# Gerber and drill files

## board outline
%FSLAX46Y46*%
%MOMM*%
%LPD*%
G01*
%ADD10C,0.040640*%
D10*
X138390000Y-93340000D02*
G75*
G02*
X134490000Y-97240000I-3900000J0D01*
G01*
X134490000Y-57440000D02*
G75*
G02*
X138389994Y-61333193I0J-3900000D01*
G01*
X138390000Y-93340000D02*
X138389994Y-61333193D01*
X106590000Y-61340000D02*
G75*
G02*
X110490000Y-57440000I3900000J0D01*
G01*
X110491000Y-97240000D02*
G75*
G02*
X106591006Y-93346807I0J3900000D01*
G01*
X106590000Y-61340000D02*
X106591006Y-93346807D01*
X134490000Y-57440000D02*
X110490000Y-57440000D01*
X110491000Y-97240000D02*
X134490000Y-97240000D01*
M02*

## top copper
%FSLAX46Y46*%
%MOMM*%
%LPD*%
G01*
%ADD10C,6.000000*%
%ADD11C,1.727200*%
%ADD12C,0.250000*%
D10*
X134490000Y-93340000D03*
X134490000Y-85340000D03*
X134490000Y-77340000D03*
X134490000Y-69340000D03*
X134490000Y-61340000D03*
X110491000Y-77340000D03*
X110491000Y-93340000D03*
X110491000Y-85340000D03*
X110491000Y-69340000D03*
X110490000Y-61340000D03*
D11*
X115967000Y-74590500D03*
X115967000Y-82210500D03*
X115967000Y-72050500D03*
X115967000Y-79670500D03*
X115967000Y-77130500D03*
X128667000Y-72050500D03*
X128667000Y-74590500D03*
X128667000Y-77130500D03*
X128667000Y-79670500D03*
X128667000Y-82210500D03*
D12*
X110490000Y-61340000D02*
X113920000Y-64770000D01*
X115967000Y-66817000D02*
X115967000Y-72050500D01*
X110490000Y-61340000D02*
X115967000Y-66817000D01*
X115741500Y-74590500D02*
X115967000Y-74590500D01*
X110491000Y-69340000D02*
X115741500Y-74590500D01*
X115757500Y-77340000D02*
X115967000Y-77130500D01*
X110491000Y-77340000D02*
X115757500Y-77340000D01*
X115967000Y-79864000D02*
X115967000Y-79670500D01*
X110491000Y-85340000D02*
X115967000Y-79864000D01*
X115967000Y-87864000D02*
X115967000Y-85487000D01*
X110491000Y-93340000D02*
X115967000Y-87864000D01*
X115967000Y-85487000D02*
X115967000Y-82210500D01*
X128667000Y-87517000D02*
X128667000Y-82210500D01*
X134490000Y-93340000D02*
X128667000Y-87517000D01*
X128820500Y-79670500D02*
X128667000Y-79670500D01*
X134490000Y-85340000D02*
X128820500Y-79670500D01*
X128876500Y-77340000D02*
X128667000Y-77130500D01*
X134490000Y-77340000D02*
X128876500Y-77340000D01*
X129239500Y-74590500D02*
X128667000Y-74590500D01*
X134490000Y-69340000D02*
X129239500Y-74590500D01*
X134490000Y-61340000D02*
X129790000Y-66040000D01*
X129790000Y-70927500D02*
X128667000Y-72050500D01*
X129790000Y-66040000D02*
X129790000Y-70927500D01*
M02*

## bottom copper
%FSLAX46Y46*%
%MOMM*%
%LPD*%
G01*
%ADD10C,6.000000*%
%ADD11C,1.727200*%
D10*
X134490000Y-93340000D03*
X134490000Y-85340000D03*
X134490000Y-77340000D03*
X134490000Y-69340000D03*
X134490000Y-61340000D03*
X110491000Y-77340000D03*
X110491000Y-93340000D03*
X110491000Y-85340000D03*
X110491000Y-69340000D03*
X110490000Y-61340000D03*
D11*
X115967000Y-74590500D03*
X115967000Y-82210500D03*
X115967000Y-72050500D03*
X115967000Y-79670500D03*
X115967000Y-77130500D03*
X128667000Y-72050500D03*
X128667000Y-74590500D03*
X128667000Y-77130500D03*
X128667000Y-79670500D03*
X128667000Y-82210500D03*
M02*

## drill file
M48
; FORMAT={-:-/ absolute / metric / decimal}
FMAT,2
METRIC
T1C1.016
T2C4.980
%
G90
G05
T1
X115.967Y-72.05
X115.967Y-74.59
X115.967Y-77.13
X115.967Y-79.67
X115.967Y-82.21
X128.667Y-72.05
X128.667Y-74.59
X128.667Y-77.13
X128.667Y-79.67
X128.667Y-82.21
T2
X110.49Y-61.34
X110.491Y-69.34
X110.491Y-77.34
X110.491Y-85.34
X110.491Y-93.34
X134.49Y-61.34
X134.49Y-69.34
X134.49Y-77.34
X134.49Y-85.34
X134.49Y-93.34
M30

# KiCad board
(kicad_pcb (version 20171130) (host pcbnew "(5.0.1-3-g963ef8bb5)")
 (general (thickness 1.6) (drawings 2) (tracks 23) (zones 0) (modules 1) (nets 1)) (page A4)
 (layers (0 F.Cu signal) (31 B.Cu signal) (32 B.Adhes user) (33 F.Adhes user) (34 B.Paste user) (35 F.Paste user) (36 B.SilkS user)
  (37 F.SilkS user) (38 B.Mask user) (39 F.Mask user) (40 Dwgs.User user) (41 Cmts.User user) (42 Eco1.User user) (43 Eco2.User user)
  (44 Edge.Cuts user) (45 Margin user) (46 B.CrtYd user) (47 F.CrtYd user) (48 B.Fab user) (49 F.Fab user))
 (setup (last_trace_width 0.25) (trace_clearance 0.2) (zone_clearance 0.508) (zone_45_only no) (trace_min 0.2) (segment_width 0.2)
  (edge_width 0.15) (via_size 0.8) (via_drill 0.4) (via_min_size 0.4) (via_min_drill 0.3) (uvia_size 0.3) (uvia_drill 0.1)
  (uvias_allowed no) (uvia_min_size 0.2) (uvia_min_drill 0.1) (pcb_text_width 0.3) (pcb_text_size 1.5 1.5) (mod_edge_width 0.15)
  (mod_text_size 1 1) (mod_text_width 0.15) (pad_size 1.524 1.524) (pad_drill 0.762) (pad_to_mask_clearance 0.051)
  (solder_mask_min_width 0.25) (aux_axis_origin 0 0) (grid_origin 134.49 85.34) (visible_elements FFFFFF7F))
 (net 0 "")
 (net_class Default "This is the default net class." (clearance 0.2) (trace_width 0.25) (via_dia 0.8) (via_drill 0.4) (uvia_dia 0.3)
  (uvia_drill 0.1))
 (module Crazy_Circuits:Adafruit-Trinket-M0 (layer F.Cu) (at 110.49 53.34)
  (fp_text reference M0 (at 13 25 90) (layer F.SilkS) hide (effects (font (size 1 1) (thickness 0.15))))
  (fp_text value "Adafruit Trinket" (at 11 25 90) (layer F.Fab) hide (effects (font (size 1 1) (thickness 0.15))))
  (fp_arc (start 24 40) (end 27.9 40) (angle 90) (layer Edge.Cuts) (width 0.04064))
  (fp_arc (start 24 8) (end 24 4.1) (angle 89.89999678) (layer Edge.Cuts) (width 0.04064))
  (fp_line (start 27.9 40) (end 27.899994 7.993193) (layer Edge.Cuts) (width 0.04064))
  (fp_arc (start 0 8) (end -3.9 8) (angle 90) (layer Edge.Cuts) (width 0.04064))
  (fp_arc (start 0.001 40) (end 0.001 43.9) (angle 89.89999678) (layer Edge.Cuts) (width 0.04064))
  (fp_line (start -3.9 8) (end -3.898994 40.006807) (layer Edge.Cuts) (width 0.04064))
  (fp_line (start 24 4.1) (end 0 4.1) (layer Edge.Cuts) (width 0.04064))
  (fp_line (start 0.001 43.9) (end 24 43.9) (layer Edge.Cuts) (width 0.04064))
  (pad Bat thru_hole circle (at 24 40 90) (size 6 6) (drill 4.98) (layers *.Cu *.Mask))
  (pad Gnd thru_hole circle (at 24 32 90) (size 6 6) (drill 4.98) (layers *.Cu *.Mask))
  (pad 4 thru_hole circle (at 24 24 90) (size 6 6) (drill 4.98) (layers *.Cu *.Mask))
  (pad 3 thru_hole circle (at 24 16 90) (size 6 6) (drill 4.98) (layers *.Cu *.Mask))
  (pad Rst thru_hole circle (at 24 8 90) (size 6 6) (drill 4.98) (layers *.Cu *.Mask))
  (pad 1 thru_hole circle (at 0.001 24 90) (size 6 6) (drill 4.98) (layers *.Cu *.Mask))
  (pad USB thru_hole circle (at 0.001 40 90) (size 6 6) (drill 4.98) (layers *.Cu *.Mask))
  (pad 0 thru_hole circle (at 0.001 32 90) (size 6 6) (drill 4.98) (layers *.Cu *.Mask))
  (pad 2 thru_hole circle (at 0.001 16 90) (size 6 6) (drill 4.98) (layers *.Cu *.Mask))
  (pad 3V thru_hole circle (at 0 8 90) (size 6 6) (drill 4.98) (layers *.Cu *.Mask))
  (pad 2 thru_hole circle (at 5.477 21.2505 180) (size 1.7272 1.7272) (drill 1.016) (layers *.Cu *.Mask F.SilkS))
  (pad USB thru_hole circle (at 5.477 28.8705 180) (size 1.7272 1.7272) (drill 1.016) (layers *.Cu *.Mask F.SilkS))
  (pad 3V thru_hole circle (at 5.477 18.7105 180) (size 1.7272 1.7272) (drill 1.016) (layers *.Cu *.Mask F.SilkS))
  (pad 0 thru_hole circle (at 5.477 26.3305 180) (size 1.7272 1.7272) (drill 1.016) (layers *.Cu *.Mask F.SilkS))
  (pad 1 thru_hole circle (at 5.477 23.7905 180) (size 1.7272 1.7272) (drill 1.016) (layers *.Cu *.Mask F.SilkS))
  (pad Rst thru_hole circle (at 18.177 18.7105 180) (size 1.7272 1.7272) (drill 1.016) (layers *.Cu *.Mask F.SilkS))
  (pad 3 thru_hole circle (at 18.177 21.2505 180) (size 1.7272 1.7272) (drill 1.016) (layers *.Cu *.Mask F.SilkS))
  (pad 4 thru_hole circle (at 18.177 23.7905 180) (size 1.7272 1.7272) (drill 1.016) (layers *.Cu *.Mask F.SilkS))
  (pad Gnd thru_hole circle (at 18.177 26.3305 180) (size 1.7272 1.7272) (drill 1.016) (layers *.Cu *.Mask F.SilkS))
  (pad Bat thru_hole circle (at 18.177 28.8705 180) (size 1.7272 1.7272) (drill 1.016) (layers *.Cu *.Mask F.SilkS)))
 (segment (start 110.49 61.34) (end 113.92 64.77) (width 0.25) (layer F.Cu) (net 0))
 (segment (start 115.967 66.817) (end 115.967 72.0505) (width 0.25) (layer F.Cu) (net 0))
 (segment (start 110.49 61.34) (end 115.967 66.817) (width 0.25) (layer F.Cu) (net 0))
 (segment (start 115.7415 74.5905) (end 115.967 74.5905) (width 0.25) (layer F.Cu) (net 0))
 (segment (start 110.491 69.34) (end 115.7415 74.5905) (width 0.25) (layer F.Cu) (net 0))
 (segment (start 115.7575 77.34) (end 115.967 77.1305) (width 0.25) (layer F.Cu) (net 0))
 (segment (start 110.491 77.34) (end 115.7575 77.34) (width 0.25) (layer F.Cu) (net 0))
 (segment (start 115.967 79.864) (end 115.967 79.6705) (width 0.25) (layer F.Cu) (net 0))
 (segment (start 110.491 85.34) (end 115.967 79.864) (width 0.25) (layer F.Cu) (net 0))
 (segment (start 115.967 87.864) (end 115.967 85.487) (width 0.25) (layer F.Cu) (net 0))
 (segment (start 110.491 93.34) (end 115.967 87.864) (width 0.25) (layer F.Cu) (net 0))
 (segment (start 115.967 85.487) (end 115.967 82.2105) (width 0.25) (layer F.Cu) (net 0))
 (segment (start 128.667 87.517) (end 128.667 82.2105) (width 0.25) (layer F.Cu) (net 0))
 (segment (start 134.49 93.34) (end 128.667 87.517) (width 0.25) (layer F.Cu) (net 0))
 (segment (start 128.8205 79.6705) (end 128.667 79.6705) (width 0.25) (layer F.Cu) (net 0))
 (segment (start 134.49 85.34) (end 128.8205 79.6705) (width 0.25) (layer F.Cu) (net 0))
 (segment (start 128.8765 77.34) (end 128.667 77.1305) (width 0.25) (layer F.Cu) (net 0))
 (segment (start 134.49 77.34) (end 128.8765 77.34) (width 0.25) (layer F.Cu) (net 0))
 (segment (start 129.2395 74.5905) (end 128.667 74.5905) (width 0.25) (layer F.Cu) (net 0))
 (segment (start 134.49 69.34) (end 129.2395 74.5905) (width 0.25) (layer F.Cu) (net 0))
 (segment (start 134.49 61.34) (end 129.79 66.04) (width 0.25) (layer F.Cu) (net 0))
 (segment (start 129.79 70.9275) (end 128.667 72.0505) (width 0.25) (layer F.Cu) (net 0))
 (segment (start 129.79 66.04) (end 129.79 70.9275) (width 0.25) (layer F.Cu) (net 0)))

